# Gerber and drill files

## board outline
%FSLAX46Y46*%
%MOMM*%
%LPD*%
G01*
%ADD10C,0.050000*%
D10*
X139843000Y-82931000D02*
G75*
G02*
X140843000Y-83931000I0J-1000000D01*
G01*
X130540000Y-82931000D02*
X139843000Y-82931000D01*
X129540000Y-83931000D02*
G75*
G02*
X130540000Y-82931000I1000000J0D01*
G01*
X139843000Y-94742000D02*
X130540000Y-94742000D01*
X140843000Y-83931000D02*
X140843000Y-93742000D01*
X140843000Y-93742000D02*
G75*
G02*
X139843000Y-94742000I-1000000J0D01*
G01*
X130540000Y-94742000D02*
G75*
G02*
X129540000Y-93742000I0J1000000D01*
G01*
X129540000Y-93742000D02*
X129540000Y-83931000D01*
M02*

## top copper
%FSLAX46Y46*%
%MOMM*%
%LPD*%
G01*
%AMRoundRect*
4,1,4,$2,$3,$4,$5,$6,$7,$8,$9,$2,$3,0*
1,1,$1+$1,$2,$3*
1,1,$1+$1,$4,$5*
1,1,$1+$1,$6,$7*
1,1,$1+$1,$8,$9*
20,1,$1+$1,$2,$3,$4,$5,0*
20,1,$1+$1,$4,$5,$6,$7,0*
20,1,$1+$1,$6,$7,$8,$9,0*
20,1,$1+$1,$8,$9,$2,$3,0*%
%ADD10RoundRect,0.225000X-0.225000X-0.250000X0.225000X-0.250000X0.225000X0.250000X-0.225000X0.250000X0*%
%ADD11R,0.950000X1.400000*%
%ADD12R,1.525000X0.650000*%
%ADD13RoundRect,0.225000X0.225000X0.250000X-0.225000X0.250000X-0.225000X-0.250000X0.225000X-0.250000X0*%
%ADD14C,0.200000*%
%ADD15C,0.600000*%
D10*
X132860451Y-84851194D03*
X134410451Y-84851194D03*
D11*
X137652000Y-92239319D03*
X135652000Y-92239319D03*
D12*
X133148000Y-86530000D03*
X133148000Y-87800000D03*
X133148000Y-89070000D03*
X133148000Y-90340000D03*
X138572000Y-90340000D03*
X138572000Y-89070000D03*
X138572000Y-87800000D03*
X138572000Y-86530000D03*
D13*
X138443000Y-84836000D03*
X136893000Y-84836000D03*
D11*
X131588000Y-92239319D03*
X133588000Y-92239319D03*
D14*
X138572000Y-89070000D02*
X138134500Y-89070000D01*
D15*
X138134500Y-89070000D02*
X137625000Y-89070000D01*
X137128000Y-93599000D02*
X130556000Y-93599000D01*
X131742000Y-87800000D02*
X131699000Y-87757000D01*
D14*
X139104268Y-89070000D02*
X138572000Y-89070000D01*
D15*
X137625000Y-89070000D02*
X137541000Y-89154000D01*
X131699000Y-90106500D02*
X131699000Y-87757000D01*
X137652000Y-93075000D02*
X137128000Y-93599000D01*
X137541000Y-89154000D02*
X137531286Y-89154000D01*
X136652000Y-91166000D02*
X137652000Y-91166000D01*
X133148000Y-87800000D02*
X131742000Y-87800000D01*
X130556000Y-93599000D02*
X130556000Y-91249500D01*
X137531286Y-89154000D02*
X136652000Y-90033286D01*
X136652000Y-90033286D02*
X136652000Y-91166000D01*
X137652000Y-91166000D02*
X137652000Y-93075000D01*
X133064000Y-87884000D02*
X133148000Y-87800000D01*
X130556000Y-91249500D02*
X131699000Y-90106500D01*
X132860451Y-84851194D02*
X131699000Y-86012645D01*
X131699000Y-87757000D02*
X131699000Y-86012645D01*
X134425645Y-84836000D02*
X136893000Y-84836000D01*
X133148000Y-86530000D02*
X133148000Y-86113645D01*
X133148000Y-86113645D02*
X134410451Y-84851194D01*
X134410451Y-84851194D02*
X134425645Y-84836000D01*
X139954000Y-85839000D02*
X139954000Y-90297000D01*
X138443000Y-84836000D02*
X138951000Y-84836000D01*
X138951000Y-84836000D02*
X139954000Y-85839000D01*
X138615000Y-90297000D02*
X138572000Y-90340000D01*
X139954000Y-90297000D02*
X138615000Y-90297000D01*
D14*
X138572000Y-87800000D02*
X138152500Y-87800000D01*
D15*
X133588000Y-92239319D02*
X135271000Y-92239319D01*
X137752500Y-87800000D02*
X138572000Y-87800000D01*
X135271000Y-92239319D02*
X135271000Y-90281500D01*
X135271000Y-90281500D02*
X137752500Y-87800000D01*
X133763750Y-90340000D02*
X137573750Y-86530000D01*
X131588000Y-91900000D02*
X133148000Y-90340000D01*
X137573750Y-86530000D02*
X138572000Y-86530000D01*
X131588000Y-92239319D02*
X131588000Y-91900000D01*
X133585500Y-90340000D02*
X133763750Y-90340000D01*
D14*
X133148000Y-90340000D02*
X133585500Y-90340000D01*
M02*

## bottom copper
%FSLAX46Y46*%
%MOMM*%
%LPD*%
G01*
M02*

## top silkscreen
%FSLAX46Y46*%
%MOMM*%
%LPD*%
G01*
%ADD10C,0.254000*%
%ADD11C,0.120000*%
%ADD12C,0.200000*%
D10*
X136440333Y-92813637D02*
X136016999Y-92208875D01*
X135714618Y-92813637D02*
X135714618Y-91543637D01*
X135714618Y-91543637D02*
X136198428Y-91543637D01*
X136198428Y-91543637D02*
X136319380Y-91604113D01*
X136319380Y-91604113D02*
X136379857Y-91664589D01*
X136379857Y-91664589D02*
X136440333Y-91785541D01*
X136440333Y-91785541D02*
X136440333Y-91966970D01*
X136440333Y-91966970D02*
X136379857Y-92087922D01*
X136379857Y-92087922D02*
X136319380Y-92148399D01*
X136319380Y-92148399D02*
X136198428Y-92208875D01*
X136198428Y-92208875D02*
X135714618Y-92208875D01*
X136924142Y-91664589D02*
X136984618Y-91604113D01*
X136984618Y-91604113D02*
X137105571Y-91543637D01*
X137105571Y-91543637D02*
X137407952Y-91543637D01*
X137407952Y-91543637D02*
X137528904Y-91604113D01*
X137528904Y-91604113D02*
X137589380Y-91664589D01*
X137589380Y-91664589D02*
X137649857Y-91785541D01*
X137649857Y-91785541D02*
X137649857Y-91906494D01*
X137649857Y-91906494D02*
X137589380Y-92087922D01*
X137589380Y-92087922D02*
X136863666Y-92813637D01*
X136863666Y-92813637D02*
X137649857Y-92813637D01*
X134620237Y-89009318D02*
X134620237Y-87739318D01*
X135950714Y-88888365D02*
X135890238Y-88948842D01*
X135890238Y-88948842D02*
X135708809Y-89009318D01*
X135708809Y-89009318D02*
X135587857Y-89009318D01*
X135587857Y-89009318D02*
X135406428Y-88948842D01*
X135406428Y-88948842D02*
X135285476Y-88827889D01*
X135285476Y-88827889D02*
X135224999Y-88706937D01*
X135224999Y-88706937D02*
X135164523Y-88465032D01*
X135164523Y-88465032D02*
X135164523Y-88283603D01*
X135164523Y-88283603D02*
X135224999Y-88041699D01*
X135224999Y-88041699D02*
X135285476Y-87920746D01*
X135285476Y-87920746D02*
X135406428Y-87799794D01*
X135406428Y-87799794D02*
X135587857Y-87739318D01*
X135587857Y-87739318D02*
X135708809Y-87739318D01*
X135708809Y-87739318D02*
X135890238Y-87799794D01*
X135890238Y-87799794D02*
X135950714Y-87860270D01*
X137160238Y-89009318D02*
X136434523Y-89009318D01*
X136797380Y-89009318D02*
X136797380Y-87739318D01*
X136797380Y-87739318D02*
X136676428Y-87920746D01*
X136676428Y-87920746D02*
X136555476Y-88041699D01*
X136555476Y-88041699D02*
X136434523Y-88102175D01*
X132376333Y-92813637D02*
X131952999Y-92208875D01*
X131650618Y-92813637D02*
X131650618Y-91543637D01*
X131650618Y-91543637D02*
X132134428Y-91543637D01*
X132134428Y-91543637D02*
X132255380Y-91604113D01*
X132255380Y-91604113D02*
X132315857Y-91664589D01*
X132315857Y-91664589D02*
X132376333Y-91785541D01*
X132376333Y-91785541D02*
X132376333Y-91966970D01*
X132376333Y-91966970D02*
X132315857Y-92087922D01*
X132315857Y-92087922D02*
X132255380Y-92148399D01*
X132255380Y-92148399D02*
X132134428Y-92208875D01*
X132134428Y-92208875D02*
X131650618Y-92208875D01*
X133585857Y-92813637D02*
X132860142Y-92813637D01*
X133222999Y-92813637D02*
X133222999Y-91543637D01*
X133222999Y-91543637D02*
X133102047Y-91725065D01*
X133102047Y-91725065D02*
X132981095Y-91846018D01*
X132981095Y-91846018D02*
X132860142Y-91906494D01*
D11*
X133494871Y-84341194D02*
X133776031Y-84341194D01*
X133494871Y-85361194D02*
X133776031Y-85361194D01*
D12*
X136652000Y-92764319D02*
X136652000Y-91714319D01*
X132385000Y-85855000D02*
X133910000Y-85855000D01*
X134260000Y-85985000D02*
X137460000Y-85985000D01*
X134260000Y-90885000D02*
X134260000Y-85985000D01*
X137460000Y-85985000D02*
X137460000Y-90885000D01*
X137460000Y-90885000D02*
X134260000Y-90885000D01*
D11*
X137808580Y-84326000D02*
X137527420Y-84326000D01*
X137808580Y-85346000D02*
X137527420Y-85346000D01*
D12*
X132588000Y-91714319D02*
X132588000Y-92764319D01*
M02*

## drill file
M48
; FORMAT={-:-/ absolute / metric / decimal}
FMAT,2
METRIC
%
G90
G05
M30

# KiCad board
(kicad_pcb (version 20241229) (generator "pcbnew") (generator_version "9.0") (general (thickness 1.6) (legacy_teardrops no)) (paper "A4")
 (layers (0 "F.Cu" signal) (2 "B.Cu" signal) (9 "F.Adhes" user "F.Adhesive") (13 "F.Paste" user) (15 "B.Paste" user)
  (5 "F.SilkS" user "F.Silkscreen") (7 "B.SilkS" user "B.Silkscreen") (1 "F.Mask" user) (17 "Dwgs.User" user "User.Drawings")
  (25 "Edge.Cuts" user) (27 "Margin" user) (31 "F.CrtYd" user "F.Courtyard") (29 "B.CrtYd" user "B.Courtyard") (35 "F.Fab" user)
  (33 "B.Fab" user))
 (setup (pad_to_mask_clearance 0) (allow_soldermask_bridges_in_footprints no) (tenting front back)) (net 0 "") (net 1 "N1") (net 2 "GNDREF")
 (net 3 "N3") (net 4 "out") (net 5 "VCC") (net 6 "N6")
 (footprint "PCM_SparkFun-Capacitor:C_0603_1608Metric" (layer "F.Cu") (at 133.635451 84.851194)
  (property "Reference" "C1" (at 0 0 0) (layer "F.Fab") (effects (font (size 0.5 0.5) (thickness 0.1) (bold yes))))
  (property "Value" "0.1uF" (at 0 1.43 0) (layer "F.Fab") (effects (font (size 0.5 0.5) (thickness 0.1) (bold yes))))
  (fp_line (start -0.14058 -0.51) (end 0.14058 -0.51) (stroke (width 0.12) (type solid)) (layer "F.SilkS"))
  (fp_line (start -0.14058 0.51) (end 0.14058 0.51) (stroke (width 0.12) (type solid)) (layer "F.SilkS"))
  (pad "1" smd roundrect (at -0.775 0) (size 0.9 0.95) (layers "F.Cu" "F.Mask" "F.Paste") (roundrect_rratio 0.25) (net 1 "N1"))
  (pad "2" smd roundrect (at 0.775 0) (size 0.9 0.95) (layers "F.Cu" "F.Mask" "F.Paste") (roundrect_rratio 0.25) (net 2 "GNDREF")))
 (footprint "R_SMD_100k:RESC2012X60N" (layer "F.Cu") (at 136.652 92.239319 180)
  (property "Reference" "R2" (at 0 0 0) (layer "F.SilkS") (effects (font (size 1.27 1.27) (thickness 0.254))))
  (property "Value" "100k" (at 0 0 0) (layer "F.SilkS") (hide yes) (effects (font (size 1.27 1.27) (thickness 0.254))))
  (fp_line (start 0 -0.525) (end 0 0.525) (stroke (width 0.2) (type solid)) (layer "F.SilkS"))
  (pad "1" smd rect (at -1 0 180) (size 0.95 1.4) (layers "F.Cu" "F.Mask" "F.Paste") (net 1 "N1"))
  (pad "2" smd rect (at 1 0 180) (size 0.95 1.4) (layers "F.Cu" "F.Mask" "F.Paste") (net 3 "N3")))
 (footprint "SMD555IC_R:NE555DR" (layer "F.Cu") (at 135.86 88.435)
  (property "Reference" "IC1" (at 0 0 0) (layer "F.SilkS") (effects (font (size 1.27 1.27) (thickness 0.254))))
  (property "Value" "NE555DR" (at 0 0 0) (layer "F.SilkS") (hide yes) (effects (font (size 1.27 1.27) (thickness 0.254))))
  (fp_line (start -3.475 -2.58) (end -1.95 -2.58) (stroke (width 0.2) (type solid)) (layer "F.SilkS"))
  (fp_line (start -1.6 -2.45) (end 1.6 -2.45) (stroke (width 0.2) (type solid)) (layer "F.SilkS"))
  (fp_line (start -1.6 2.45) (end -1.6 -2.45) (stroke (width 0.2) (type solid)) (layer "F.SilkS"))
  (fp_line (start 1.6 -2.45) (end 1.6 2.45) (stroke (width 0.2) (type solid)) (layer "F.SilkS"))
  (fp_line (start 1.6 2.45) (end -1.6 2.45) (stroke (width 0.2) (type solid)) (layer "F.SilkS"))
  (pad "1" smd rect (at -2.712 -1.905 90) (size 0.65 1.525) (layers "F.Cu" "F.Paste") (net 2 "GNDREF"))
  (pad "2" smd rect (at -2.712 -0.635 90) (size 0.65 1.525) (layers "F.Cu" "F.Paste") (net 1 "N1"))
  (pad "3" smd rect (at -2.712 0.635 90) (size 0.65 1.525) (layers "F.Cu" "F.Paste") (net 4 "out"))
  (pad "4" smd rect (at -2.712 1.905 90) (size 0.65 1.525) (layers "F.Cu" "F.Paste") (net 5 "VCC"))
  (pad "5" smd rect (at 2.712 1.905 90) (size 0.65 1.525) (layers "F.Cu" "F.Paste") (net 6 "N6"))
  (pad "6" smd rect (at 2.712 0.635 90) (size 0.65 1.525) (layers "F.Cu" "F.Paste") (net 1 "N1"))
  (pad "7" smd rect (at 2.712 -0.635 90) (size 0.65 1.525) (layers "F.Cu" "F.Paste") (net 3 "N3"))
  (pad "8" smd rect (at 2.712 -1.905 90) (size 0.65 1.525) (layers "F.Cu" "F.Paste") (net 5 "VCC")))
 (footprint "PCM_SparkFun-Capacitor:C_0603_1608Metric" (layer "F.Cu") (at 137.668 84.836 180)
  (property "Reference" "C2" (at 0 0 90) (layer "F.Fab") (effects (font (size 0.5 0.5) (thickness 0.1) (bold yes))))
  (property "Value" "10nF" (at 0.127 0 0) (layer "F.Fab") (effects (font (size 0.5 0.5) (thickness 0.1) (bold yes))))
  (fp_line (start -0.14058 0.51) (end 0.14058 0.51) (stroke (width 0.12) (type solid)) (layer "F.SilkS"))
  (fp_line (start -0.14058 -0.51) (end 0.14058 -0.51) (stroke (width 0.12) (type solid)) (layer "F.SilkS"))
  (pad "1" smd roundrect (at -0.775 0 180) (size 0.9 0.95) (layers "F.Cu" "F.Mask" "F.Paste") (roundrect_rratio 0.25) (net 6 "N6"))
  (pad "2" smd roundrect (at 0.775 0 180) (size 0.9 0.95) (layers "F.Cu" "F.Mask" "F.Paste") (roundrect_rratio 0.25) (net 2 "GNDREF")))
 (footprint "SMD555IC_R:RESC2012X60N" (layer "F.Cu") (at 132.588 92.239319)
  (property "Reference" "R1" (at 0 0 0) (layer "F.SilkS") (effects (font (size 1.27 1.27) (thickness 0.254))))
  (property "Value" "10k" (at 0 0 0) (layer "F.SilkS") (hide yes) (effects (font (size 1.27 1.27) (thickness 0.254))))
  (fp_line (start 0 -0.525) (end 0 0.525) (stroke (width 0.2) (type solid)) (layer "F.SilkS"))
  (pad "1" smd rect (at -1 0) (size 0.95 1.4) (layers "F.Cu" "F.Mask" "F.Paste") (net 5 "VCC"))
  (pad "2" smd rect (at 1 0) (size 0.95 1.4) (layers "F.Cu" "F.Mask" "F.Paste") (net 3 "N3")))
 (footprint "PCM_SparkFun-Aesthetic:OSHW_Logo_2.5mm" (layer "B.Cu") (at 139.192 84.709 180)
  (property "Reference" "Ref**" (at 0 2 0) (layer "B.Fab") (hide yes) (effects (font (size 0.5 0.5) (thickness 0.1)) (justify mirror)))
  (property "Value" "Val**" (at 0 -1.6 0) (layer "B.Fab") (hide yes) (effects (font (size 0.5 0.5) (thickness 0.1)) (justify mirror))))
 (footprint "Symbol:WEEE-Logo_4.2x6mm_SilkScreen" (layer "B.Cu") (at 132.08 91.44 180)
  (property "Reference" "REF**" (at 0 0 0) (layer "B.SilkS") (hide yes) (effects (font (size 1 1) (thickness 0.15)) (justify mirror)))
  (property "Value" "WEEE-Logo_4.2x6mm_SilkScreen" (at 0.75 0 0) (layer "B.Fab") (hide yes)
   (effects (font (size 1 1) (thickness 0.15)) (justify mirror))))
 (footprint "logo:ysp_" (layer "B.Cu") (at 137.922 88.519 180)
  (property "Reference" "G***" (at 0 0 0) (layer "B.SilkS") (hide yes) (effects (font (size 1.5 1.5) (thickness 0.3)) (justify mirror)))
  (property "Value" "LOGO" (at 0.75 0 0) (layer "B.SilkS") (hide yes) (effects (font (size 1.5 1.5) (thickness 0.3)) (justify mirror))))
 (gr_arc (start 139.843 82.931) (mid 140.550107 83.223893) (end 140.843 83.931) (stroke (width 0.05) (type default)) (layer "Edge.Cuts"))
 (gr_line (start 130.54 82.931) (end 139.843 82.931) (stroke (width 0.05) (type default)) (layer "Edge.Cuts"))
 (gr_arc (start 129.54 83.931) (mid 129.832893 83.223893) (end 130.54 82.931) (stroke (width 0.05) (type default)) (layer "Edge.Cuts"))
 (gr_line (start 139.843 94.742) (end 130.54 94.742) (stroke (width 0.05) (type default)) (layer "Edge.Cuts"))
 (gr_line (start 140.843 83.931) (end 140.843 93.742) (stroke (width 0.05) (type default)) (layer "Edge.Cuts"))
 (gr_arc (start 140.843 93.742) (mid 140.550107 94.449107) (end 139.843 94.742) (stroke (width 0.05) (type default)) (layer "Edge.Cuts"))
 (gr_arc (start 130.54 94.742) (mid 129.832893 94.449107) (end 129.54 93.742) (stroke (width 0.05) (type default)) (layer "Edge.Cuts"))
 (gr_line (start 129.54 93.742) (end 129.54 83.931) (stroke (width 0.05) (type default)) (layer "Edge.Cuts"))
 (segment (start 138.572 89.07) (end 138.1345 89.07) (width 0.2) (layer "F.Cu") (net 1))
 (segment (start 138.1345 89.07) (end 137.625 89.07) (width 0.6) (layer "F.Cu") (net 1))
 (segment (start 137.128 93.599) (end 130.556 93.599) (width 0.6) (layer "F.Cu") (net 1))
 (segment (start 131.742 87.8) (end 131.699 87.757) (width 0.6) (layer "F.Cu") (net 1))
 (segment (start 139.104268 89.07) (end 138.572 89.07) (width 0.2) (layer "F.Cu") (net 1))
 (segment (start 137.625 89.07) (end 137.541 89.154) (width 0.6) (layer "F.Cu") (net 1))
 (segment (start 131.699 90.1065) (end 131.699 87.757) (width 0.6) (layer "F.Cu") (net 1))
 (segment (start 137.652 93.075) (end 137.128 93.599) (width 0.6) (layer "F.Cu") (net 1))
 (segment (start 137.541 89.154) (end 137.531286 89.154) (width 0.6) (layer "F.Cu") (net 1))
 (segment (start 136.652 91.166) (end 137.652 91.166) (width 0.6) (layer "F.Cu") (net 1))
 (segment (start 133.148 87.8) (end 131.742 87.8) (width 0.6) (layer "F.Cu") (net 1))
 (segment (start 130.556 93.599) (end 130.556 91.2495) (width 0.6) (layer "F.Cu") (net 1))
 (segment (start 137.531286 89.154) (end 136.652 90.033286) (width 0.6) (layer "F.Cu") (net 1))
 (segment (start 136.652 90.033286) (end 136.652 91.166) (width 0.6) (layer "F.Cu") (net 1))
 (segment (start 137.652 91.166) (end 137.652 93.075) (width 0.6) (layer "F.Cu") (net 1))
 (segment (start 133.064 87.884) (end 133.148 87.8) (width 0.6) (layer "F.Cu") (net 1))
 (segment (start 130.556 91.2495) (end 131.699 90.1065) (width 0.6) (layer "F.Cu") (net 1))
 (segment (start 132.860451 84.851194) (end 131.699 86.012645) (width 0.6) (layer "F.Cu") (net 1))
 (segment (start 131.699 87.757) (end 131.699 86.012645) (width 0.6) (layer "F.Cu") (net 1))
 (segment (start 134.425645 84.836) (end 136.893 84.836) (width 0.6) (layer "F.Cu") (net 2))
 (segment (start 133.148 86.53) (end 133.148 86.113645) (width 0.6) (layer "F.Cu") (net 2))
 (segment (start 133.148 86.113645) (end 134.410451 84.851194) (width 0.6) (layer "F.Cu") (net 2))
 (segment (start 134.410451 84.851194) (end 134.425645 84.836) (width 0.6) (layer "F.Cu") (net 2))
 (segment (start 139.954 85.839) (end 139.954 90.297) (width 0.6) (layer "F.Cu") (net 6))
 (segment (start 138.443 84.836) (end 138.951 84.836) (width 0.6) (layer "F.Cu") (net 6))
 (segment (start 138.951 84.836) (end 139.954 85.839) (width 0.6) (layer "F.Cu") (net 6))
 (segment (start 138.615 90.297) (end 138.572 90.34) (width 0.6) (layer "F.Cu") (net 6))
 (segment (start 139.954 90.297) (end 138.615 90.297) (width 0.6) (layer "F.Cu") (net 6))
 (segment (start 138.572 87.8) (end 138.1525 87.8) (width 0.2) (layer "F.Cu") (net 3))
 (segment (start 133.588 92.239319) (end 135.271 92.239319) (width 0.6) (layer "F.Cu") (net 3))
 (segment (start 137.7525 87.8) (end 138.572 87.8) (width 0.6) (layer "F.Cu") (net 3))
 (segment (start 135.271 92.239319) (end 135.271 90.2815) (width 0.6) (layer "F.Cu") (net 3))
 (segment (start 135.271 90.2815) (end 137.7525 87.8) (width 0.6) (layer "F.Cu") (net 3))
 (segment (start 133.76375 90.34) (end 137.57375 86.53) (width 0.6) (layer "F.Cu") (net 5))
 (segment (start 131.588 91.9) (end 133.148 90.34) (width 0.6) (layer "F.Cu") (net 5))
 (segment (start 137.57375 86.53) (end 138.572 86.53) (width 0.6) (layer "F.Cu") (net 5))
 (segment (start 131.588 92.239319) (end 131.588 91.9) (width 0.6) (layer "F.Cu") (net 5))
 (segment (start 133.5855 90.34) (end 133.76375 90.34) (width 0.6) (layer "F.Cu") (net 5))
 (segment (start 133.148 90.34) (end 133.5855 90.34) (width 0.2) (layer "F.Cu") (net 5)))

